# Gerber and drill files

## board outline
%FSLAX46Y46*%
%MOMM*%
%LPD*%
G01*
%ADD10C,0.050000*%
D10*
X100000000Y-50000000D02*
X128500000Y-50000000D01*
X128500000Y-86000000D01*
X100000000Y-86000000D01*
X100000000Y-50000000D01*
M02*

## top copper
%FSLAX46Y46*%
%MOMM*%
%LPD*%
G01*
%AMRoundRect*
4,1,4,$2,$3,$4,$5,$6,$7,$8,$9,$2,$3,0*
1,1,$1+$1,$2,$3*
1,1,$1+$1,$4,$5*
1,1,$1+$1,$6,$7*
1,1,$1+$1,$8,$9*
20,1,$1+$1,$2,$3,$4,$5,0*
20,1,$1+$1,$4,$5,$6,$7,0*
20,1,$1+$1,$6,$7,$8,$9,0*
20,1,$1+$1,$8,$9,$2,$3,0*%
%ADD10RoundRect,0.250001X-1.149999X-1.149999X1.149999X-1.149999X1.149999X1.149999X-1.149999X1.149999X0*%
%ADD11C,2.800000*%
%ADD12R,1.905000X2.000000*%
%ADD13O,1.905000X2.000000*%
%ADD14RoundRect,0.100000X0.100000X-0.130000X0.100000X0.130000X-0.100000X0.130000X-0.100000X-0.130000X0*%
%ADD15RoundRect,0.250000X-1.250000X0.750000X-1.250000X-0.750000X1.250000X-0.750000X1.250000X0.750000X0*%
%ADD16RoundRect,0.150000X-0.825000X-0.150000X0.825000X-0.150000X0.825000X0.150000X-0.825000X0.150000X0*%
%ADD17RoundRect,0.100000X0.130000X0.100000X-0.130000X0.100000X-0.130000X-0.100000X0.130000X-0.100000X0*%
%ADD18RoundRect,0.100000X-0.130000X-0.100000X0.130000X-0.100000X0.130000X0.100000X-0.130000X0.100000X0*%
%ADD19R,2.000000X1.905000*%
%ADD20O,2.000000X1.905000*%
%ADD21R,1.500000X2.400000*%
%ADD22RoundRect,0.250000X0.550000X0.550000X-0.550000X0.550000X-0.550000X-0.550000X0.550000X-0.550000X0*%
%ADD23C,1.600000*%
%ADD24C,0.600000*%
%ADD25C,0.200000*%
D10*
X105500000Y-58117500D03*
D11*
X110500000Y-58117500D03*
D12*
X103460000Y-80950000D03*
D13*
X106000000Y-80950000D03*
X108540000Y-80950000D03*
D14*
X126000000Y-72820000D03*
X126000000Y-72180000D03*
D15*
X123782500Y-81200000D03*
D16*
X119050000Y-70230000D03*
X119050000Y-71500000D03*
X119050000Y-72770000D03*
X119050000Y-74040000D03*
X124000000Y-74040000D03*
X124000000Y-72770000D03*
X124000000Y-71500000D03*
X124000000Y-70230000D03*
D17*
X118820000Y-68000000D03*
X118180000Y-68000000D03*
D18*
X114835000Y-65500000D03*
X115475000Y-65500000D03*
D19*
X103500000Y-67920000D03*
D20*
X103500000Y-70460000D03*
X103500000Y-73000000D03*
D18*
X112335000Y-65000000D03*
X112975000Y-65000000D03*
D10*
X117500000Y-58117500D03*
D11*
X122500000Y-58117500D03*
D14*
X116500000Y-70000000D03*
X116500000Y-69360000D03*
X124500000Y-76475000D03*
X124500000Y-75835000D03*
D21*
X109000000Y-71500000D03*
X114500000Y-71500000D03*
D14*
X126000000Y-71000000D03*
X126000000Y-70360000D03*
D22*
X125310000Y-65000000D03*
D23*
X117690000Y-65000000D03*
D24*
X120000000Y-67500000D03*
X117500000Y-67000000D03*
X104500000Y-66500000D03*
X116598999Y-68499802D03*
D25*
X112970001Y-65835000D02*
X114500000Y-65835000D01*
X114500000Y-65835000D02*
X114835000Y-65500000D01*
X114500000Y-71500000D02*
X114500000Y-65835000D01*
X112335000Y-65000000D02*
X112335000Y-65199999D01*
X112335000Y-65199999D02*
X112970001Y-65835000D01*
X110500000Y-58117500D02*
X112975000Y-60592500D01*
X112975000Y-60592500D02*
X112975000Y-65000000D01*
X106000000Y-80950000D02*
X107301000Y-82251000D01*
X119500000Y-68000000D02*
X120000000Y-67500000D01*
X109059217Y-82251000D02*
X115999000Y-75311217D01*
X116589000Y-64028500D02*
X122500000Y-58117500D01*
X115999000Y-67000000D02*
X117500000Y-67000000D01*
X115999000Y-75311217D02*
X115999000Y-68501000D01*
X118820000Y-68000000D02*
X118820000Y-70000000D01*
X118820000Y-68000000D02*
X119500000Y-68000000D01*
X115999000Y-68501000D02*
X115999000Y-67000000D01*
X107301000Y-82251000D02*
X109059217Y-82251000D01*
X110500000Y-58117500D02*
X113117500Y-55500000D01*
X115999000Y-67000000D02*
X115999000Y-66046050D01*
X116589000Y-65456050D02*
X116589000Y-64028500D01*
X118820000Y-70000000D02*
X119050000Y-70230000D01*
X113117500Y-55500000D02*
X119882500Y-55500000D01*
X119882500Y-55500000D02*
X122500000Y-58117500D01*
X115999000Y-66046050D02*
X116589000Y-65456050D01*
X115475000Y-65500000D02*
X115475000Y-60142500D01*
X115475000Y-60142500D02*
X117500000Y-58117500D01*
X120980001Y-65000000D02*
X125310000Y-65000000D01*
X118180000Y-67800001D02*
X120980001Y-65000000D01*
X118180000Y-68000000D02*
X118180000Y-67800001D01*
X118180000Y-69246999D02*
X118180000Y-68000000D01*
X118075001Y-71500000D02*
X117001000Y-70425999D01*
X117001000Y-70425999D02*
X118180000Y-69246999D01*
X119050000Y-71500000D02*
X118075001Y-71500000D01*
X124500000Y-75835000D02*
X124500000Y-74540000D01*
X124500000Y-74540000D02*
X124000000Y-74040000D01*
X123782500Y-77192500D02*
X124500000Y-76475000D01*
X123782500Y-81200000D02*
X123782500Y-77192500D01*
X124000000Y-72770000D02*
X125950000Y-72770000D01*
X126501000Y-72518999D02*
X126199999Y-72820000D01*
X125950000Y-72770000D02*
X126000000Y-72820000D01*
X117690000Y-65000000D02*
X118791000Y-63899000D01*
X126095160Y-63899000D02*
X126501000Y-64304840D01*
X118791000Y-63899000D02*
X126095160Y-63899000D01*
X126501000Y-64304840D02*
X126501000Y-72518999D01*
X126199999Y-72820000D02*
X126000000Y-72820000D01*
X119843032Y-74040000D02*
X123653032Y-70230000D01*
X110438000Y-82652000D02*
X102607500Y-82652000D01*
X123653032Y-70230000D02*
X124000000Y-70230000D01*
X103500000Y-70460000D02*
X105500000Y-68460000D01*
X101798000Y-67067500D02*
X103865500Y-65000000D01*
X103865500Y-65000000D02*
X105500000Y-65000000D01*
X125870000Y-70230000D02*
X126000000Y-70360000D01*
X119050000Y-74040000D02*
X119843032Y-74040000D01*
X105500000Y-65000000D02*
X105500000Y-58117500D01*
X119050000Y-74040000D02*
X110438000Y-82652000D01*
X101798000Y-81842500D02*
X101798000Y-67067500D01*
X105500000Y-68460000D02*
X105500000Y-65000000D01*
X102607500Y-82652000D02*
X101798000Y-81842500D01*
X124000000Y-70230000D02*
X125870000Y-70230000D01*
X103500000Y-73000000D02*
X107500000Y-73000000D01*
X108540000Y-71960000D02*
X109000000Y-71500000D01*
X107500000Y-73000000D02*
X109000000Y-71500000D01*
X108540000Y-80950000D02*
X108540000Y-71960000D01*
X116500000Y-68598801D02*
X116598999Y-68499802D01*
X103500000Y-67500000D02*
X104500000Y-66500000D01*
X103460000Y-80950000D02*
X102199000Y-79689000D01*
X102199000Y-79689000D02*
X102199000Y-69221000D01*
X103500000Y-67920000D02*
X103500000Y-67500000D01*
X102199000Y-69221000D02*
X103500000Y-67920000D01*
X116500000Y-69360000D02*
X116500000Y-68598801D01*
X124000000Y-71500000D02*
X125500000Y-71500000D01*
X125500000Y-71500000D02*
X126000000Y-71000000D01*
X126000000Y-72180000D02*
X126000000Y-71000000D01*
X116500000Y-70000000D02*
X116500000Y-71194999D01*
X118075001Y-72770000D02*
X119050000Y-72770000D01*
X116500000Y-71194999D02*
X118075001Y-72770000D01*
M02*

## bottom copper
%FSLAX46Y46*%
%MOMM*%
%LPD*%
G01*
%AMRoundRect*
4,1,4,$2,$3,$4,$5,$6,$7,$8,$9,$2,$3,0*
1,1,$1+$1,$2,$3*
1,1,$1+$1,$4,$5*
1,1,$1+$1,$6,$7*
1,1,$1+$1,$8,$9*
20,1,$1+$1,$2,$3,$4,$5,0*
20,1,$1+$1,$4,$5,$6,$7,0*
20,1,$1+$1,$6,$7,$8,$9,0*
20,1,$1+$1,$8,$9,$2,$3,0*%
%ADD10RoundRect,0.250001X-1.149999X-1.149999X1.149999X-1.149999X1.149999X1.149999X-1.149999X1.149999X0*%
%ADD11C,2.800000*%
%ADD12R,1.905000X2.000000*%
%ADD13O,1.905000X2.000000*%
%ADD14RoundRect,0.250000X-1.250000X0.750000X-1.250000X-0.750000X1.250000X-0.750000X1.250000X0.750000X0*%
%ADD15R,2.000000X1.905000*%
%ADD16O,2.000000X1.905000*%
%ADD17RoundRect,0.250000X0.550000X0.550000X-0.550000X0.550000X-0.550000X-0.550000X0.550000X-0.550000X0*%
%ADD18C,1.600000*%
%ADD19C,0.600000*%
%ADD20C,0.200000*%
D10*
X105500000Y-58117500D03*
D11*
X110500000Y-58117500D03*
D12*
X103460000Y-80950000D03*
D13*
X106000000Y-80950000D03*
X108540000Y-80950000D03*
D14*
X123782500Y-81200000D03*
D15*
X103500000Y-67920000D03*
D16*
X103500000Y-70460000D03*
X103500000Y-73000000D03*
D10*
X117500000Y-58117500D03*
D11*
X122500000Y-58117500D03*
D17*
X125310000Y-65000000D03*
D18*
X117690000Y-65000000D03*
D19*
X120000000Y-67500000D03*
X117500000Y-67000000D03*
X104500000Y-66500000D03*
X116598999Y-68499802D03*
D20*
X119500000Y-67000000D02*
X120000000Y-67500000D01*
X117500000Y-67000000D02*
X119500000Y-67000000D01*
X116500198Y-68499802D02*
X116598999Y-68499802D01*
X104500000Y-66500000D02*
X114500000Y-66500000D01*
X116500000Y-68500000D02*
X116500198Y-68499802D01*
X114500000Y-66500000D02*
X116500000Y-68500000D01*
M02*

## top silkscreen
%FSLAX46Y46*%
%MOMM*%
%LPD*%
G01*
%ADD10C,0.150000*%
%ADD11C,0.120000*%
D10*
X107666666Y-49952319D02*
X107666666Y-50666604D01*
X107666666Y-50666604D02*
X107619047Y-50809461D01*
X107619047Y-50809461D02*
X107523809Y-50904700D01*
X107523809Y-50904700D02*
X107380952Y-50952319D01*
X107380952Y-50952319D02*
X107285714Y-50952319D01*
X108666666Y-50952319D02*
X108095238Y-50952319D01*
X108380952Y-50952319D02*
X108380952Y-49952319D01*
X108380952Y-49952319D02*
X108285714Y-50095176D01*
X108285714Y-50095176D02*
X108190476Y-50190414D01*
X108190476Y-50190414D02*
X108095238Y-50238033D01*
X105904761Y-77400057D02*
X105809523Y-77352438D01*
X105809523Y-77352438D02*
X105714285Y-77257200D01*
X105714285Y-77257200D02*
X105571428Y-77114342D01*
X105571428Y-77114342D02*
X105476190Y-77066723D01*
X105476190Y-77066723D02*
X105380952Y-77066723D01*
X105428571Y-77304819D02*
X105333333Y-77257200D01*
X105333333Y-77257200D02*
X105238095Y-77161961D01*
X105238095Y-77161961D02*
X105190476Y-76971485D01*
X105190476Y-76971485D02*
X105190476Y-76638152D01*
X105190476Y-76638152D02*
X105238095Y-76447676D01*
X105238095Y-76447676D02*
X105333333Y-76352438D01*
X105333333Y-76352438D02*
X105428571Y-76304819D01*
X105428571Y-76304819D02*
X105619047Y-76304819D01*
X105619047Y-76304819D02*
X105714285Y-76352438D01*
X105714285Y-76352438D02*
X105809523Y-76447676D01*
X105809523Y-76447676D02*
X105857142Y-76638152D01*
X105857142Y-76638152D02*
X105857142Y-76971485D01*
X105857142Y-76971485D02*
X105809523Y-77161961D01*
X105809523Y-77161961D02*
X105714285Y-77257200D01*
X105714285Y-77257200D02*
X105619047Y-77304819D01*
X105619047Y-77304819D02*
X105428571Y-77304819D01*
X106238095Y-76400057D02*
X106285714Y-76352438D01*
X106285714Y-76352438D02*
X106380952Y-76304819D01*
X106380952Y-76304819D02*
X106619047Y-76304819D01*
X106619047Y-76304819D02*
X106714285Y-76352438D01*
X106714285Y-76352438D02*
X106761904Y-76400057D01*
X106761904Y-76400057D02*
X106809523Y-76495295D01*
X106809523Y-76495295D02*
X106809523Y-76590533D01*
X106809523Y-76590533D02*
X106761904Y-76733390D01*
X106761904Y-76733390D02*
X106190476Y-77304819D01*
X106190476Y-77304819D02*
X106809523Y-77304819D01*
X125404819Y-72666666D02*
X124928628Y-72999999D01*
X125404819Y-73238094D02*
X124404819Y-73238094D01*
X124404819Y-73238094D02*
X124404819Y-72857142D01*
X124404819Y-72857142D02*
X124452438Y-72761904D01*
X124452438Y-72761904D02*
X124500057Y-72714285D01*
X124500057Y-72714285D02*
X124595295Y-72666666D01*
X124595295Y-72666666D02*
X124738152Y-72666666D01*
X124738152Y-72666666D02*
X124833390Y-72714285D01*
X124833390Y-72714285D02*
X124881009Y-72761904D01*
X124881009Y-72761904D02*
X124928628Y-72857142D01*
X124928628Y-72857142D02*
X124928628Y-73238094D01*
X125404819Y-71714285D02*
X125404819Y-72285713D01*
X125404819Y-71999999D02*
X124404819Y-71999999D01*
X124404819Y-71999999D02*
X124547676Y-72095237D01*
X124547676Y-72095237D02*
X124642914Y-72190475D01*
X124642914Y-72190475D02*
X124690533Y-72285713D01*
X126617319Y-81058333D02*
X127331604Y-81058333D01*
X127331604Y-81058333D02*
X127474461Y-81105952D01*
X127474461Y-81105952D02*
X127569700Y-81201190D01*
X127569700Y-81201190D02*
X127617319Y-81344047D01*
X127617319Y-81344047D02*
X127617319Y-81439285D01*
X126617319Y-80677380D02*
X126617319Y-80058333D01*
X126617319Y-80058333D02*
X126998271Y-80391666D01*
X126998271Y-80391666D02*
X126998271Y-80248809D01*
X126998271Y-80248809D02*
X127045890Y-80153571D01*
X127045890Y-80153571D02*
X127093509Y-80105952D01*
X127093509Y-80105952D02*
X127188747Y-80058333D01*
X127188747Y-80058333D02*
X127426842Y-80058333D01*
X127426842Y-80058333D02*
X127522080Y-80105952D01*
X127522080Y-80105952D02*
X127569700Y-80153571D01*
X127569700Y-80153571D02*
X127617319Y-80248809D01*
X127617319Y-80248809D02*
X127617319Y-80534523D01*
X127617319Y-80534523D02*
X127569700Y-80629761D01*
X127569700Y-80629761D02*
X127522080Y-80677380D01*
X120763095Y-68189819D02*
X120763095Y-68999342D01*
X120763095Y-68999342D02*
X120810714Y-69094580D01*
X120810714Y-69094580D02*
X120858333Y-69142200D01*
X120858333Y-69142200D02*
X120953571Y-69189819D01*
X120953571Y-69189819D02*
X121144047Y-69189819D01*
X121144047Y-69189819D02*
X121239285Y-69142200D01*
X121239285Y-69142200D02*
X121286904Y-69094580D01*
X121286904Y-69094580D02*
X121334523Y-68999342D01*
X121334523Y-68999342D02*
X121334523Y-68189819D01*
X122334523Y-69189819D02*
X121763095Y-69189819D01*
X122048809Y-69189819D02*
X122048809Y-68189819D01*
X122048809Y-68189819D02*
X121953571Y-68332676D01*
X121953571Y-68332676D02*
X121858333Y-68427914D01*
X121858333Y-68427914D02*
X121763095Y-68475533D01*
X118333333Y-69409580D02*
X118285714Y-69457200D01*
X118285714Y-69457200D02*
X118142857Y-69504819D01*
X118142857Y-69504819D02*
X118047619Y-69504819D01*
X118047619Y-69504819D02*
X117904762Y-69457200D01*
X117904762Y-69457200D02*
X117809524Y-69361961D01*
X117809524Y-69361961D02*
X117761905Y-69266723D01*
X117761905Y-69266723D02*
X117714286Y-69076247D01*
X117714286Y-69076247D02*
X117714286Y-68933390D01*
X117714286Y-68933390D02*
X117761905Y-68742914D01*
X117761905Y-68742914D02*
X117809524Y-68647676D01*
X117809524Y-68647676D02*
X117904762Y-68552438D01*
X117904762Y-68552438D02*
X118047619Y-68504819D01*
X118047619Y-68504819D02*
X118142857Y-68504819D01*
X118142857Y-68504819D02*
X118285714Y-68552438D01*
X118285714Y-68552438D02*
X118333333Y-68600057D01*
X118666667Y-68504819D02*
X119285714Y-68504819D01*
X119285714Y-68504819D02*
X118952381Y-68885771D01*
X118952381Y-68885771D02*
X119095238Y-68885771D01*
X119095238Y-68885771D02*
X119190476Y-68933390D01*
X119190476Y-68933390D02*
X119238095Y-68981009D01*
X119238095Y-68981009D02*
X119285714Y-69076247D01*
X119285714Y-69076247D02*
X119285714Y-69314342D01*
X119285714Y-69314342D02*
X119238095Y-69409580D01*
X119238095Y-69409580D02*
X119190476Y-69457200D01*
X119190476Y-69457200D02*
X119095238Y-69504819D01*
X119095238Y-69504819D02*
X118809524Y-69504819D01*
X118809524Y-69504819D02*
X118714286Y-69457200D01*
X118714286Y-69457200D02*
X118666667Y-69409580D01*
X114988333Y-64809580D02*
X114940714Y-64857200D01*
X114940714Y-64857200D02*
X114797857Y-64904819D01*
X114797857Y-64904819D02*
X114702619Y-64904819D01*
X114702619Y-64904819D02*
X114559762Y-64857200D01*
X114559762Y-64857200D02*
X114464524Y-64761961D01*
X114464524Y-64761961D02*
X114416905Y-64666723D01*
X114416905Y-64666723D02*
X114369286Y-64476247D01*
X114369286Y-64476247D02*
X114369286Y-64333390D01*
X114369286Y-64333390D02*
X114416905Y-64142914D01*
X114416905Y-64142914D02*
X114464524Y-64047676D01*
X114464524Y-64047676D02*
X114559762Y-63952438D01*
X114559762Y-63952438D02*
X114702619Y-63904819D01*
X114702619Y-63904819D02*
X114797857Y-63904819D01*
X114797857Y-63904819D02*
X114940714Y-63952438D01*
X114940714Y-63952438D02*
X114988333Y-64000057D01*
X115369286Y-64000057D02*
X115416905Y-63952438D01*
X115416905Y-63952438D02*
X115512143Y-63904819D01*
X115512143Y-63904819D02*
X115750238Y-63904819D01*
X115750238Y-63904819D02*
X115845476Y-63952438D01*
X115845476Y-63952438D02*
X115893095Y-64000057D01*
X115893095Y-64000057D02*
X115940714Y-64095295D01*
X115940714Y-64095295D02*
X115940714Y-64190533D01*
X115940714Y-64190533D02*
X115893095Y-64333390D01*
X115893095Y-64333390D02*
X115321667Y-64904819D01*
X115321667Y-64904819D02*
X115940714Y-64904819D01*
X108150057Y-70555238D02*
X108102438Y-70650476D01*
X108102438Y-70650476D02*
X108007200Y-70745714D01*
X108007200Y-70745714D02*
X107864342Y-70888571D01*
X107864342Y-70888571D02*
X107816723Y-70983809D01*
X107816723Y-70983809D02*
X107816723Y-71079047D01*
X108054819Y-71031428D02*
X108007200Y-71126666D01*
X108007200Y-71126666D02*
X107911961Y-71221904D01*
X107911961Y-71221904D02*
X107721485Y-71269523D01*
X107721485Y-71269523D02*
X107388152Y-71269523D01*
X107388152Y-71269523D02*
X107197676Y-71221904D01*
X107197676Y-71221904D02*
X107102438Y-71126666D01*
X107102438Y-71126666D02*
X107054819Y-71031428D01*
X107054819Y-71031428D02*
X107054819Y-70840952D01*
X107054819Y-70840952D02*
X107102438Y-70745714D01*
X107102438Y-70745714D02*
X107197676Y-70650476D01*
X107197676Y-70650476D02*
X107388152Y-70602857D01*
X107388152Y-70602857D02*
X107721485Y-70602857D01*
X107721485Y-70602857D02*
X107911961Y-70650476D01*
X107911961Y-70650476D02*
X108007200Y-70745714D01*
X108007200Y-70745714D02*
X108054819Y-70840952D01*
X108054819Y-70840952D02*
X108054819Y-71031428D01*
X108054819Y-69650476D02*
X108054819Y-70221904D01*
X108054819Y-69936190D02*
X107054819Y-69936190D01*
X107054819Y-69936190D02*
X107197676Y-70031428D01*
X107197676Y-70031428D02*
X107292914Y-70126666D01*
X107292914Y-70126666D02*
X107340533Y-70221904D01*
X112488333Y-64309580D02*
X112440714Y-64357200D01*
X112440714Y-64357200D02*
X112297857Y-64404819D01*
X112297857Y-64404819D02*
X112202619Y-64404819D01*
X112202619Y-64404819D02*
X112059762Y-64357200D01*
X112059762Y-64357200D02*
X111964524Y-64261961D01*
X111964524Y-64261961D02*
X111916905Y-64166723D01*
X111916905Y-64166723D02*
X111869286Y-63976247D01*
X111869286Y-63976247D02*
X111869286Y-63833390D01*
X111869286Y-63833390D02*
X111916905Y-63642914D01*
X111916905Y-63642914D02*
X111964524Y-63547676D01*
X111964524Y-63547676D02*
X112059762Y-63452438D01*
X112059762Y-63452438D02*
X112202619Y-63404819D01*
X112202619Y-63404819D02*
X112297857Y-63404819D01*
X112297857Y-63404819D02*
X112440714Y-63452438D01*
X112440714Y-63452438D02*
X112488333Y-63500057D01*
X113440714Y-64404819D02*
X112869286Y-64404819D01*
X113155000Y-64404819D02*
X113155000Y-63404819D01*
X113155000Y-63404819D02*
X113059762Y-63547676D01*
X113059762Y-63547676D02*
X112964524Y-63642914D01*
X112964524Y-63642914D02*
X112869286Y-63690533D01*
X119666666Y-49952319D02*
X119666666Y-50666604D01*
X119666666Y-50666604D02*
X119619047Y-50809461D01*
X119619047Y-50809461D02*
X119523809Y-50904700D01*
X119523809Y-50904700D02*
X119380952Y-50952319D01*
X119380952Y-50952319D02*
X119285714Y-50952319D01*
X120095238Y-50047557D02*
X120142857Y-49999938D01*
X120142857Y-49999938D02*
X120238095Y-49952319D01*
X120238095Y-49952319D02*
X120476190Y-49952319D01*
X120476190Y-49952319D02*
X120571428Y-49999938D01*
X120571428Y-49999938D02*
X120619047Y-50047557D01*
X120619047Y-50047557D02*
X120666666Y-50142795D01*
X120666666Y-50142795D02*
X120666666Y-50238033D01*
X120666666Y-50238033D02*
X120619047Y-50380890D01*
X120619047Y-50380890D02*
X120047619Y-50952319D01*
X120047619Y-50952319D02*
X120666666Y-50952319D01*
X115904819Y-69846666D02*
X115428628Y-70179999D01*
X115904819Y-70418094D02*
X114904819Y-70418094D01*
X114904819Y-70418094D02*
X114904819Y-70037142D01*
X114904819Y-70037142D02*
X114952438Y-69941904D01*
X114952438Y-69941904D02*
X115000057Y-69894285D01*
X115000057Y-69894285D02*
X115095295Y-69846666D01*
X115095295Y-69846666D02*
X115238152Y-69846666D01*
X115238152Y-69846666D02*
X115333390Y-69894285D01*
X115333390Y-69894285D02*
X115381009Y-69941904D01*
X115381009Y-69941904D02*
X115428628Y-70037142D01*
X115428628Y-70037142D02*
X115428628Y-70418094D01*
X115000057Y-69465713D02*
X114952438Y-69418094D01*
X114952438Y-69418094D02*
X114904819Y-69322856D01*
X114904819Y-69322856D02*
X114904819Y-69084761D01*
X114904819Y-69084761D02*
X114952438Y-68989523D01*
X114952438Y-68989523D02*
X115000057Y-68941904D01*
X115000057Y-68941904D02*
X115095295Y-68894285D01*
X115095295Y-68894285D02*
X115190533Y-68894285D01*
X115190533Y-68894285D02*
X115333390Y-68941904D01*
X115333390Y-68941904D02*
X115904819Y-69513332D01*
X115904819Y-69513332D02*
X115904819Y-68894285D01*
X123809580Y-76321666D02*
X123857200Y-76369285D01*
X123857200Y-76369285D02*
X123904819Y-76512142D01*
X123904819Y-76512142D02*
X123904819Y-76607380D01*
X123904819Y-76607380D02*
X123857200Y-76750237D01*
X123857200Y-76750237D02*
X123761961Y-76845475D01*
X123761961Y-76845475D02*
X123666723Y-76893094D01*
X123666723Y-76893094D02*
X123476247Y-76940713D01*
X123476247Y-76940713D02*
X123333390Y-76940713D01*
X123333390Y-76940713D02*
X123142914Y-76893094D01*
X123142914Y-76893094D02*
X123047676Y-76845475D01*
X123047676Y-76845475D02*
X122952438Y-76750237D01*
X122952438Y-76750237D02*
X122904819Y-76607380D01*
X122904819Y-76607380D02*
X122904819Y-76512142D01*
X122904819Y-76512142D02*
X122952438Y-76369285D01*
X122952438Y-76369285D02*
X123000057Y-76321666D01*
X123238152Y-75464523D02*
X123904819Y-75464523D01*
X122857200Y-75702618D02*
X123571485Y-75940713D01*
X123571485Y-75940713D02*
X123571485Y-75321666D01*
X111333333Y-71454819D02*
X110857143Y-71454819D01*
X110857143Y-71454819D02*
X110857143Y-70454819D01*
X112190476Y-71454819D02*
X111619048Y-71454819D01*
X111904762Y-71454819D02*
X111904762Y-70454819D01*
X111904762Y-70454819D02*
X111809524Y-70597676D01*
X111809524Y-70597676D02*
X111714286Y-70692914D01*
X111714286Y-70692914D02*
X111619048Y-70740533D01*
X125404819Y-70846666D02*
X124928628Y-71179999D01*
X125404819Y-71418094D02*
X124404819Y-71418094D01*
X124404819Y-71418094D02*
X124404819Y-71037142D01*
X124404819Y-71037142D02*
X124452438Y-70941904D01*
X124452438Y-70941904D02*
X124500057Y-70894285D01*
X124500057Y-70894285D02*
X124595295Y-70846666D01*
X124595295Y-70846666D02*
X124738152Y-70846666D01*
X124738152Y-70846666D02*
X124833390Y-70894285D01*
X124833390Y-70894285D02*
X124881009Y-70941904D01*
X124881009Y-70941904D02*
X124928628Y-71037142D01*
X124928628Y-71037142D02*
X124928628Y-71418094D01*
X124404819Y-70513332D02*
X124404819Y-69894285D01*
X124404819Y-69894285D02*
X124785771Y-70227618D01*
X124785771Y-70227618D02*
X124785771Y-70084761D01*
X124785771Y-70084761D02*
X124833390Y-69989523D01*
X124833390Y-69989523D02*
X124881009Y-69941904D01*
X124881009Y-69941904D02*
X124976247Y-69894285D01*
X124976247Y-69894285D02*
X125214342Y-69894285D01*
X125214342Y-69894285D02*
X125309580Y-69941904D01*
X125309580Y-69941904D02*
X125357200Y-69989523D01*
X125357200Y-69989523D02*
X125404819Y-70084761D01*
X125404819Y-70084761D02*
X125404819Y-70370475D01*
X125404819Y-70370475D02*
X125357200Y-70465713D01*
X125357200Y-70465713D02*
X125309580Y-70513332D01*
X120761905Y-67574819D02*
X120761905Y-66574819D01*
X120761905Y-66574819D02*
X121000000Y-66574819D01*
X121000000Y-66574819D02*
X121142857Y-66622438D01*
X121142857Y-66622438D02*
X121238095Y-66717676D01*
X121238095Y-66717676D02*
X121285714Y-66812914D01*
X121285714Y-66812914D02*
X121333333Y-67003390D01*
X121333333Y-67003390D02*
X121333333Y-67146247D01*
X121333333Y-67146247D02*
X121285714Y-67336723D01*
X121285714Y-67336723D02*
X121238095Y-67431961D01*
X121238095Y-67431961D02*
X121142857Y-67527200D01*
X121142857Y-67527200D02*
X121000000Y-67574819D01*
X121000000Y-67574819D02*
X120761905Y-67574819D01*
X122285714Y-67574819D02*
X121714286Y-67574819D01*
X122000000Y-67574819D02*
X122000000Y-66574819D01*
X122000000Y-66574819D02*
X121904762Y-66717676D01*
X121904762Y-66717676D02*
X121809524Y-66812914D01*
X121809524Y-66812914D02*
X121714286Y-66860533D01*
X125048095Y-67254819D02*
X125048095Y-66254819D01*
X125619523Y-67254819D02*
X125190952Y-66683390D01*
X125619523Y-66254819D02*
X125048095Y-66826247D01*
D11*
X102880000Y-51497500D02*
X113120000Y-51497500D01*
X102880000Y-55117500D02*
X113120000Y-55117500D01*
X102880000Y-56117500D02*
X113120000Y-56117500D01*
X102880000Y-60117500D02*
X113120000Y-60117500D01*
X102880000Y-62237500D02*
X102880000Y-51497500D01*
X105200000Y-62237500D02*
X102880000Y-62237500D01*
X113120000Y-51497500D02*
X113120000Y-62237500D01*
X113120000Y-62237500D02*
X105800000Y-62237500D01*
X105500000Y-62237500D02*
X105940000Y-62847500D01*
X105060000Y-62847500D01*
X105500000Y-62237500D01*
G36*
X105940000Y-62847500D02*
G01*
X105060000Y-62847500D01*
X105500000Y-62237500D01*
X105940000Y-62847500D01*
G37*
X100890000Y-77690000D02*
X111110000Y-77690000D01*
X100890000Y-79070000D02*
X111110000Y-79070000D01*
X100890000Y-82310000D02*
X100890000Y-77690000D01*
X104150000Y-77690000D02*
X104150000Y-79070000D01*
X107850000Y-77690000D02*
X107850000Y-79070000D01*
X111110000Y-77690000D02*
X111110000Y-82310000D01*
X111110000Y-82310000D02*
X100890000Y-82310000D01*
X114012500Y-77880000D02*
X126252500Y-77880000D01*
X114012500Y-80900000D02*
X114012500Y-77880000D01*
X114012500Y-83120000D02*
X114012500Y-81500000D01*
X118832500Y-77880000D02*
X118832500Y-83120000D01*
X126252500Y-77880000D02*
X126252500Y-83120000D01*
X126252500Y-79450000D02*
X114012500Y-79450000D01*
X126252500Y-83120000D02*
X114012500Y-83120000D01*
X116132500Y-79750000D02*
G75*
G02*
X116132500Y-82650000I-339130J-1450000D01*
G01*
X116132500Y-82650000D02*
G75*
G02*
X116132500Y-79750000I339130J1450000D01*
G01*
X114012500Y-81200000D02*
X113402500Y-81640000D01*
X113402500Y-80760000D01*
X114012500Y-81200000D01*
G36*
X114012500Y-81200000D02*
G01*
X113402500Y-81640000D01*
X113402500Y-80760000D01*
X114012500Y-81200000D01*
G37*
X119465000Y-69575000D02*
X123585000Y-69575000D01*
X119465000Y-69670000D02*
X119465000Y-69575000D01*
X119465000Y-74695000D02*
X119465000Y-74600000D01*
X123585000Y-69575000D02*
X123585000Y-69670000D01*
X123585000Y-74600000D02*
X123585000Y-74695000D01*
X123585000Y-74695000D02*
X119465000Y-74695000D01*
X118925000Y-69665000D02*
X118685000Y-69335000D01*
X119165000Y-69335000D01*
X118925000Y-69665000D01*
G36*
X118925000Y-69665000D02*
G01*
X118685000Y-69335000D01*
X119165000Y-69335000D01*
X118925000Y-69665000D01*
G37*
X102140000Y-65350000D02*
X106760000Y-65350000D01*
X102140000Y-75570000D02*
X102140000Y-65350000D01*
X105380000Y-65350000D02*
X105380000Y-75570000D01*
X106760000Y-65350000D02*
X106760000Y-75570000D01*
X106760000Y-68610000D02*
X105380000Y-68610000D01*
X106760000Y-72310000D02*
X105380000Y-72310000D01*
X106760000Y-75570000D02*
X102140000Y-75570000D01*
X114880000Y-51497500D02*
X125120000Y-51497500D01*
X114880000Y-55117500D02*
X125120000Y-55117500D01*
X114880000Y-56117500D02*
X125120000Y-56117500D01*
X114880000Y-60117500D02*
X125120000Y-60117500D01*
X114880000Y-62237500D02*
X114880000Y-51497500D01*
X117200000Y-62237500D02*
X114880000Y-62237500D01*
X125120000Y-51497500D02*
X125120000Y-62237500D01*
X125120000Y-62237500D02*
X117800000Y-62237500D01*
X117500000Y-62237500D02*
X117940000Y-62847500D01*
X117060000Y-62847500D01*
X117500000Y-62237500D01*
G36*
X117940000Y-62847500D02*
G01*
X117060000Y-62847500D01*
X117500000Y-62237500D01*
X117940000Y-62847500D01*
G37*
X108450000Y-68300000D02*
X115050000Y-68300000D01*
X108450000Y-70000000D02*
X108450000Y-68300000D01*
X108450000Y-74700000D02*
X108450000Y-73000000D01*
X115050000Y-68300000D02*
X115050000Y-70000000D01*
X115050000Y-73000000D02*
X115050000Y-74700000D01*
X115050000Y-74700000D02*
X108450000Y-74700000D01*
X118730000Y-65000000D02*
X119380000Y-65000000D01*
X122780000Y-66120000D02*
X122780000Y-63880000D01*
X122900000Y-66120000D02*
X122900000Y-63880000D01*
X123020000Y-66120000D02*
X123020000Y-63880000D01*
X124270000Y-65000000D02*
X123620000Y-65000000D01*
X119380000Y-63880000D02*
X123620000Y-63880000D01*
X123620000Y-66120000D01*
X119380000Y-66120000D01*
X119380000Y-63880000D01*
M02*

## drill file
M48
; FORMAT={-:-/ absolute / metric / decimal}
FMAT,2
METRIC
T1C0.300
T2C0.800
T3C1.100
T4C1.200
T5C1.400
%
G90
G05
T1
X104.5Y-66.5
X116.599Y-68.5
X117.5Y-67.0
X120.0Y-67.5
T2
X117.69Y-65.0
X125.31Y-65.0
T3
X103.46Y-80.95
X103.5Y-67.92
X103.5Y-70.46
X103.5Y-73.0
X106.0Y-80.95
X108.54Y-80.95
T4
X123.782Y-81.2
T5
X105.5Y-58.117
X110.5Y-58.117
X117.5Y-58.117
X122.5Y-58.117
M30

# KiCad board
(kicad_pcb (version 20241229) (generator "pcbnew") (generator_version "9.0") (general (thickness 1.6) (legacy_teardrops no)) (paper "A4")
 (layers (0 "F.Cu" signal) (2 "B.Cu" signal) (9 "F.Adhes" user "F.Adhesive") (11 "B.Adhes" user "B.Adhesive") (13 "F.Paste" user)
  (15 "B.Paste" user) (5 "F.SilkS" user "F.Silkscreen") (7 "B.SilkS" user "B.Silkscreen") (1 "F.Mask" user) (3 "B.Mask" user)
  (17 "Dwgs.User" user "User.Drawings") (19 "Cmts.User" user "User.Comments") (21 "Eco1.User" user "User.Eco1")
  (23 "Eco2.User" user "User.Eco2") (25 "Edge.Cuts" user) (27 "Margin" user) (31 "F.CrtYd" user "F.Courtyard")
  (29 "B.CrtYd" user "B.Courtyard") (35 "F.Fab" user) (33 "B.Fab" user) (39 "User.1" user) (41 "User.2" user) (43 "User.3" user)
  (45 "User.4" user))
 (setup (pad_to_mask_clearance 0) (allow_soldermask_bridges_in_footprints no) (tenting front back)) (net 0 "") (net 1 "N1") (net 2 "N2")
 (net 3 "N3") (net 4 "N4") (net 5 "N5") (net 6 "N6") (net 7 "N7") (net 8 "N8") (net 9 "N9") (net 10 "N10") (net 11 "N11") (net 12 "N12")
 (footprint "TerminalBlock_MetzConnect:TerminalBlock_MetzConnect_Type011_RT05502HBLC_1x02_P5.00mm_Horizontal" (layer "F.Cu")
  (at 105.5 58.1175)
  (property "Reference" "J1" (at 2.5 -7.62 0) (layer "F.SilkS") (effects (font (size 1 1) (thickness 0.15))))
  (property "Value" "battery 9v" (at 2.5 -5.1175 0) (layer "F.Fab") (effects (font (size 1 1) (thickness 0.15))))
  (fp_line (start -2.62 -6.62) (end 7.62 -6.62) (stroke (width 0.12) (type solid)) (layer "F.SilkS"))
  (fp_line (start -2.62 -3) (end 7.62 -3) (stroke (width 0.12) (type solid)) (layer "F.SilkS"))
  (fp_line (start -2.62 -2) (end 7.62 -2) (stroke (width 0.12) (type solid)) (layer "F.SilkS"))
  (fp_line (start -2.62 2) (end 7.62 2) (stroke (width 0.12) (type solid)) (layer "F.SilkS"))
  (fp_line (start -2.62 4.12) (end -2.62 -6.62) (stroke (width 0.12) (type solid)) (layer "F.SilkS"))
  (fp_line (start -0.3 4.12) (end -2.62 4.12) (stroke (width 0.12) (type solid)) (layer "F.SilkS"))
  (fp_line (start 7.62 -6.62) (end 7.62 4.12) (stroke (width 0.12) (type solid)) (layer "F.SilkS"))
  (fp_line (start 7.62 4.12) (end 0.3 4.12) (stroke (width 0.12) (type solid)) (layer "F.SilkS"))
  (fp_poly (pts (xy 0 4.12) (xy 0.44 4.73) (xy -0.44 4.73)) (stroke (width 0.12) (type solid)) (fill yes) (layer "F.SilkS"))
  (pad "1" thru_hole roundrect (at 0 0) (size 2.8 2.8) (drill 1.4) (layers "*.Cu" "*.Mask") (remove_unused_layers no)
   (roundrect_rratio 0.089286) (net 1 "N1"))
  (pad "2" thru_hole circle (at 5 0) (size 2.8 2.8) (drill 1.4) (layers "*.Cu" "*.Mask") (remove_unused_layers no) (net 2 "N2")))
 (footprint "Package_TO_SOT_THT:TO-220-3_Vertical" (layer "F.Cu") (at 103.46 80.95)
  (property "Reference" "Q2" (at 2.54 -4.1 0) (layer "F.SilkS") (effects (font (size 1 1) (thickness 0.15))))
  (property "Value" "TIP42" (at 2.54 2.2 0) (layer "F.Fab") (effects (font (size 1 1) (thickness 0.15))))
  (fp_line (start -2.57 -3.26) (end 7.65 -3.26) (stroke (width 0.12) (type solid)) (layer "F.SilkS"))
  (fp_line (start -2.57 -1.88) (end 7.65 -1.88) (stroke (width 0.12) (type solid)) (layer "F.SilkS"))
  (fp_line (start -2.57 1.36) (end -2.57 -3.26) (stroke (width 0.12) (type solid)) (layer "F.SilkS"))
  (fp_line (start 0.69 -3.26) (end 0.69 -1.88) (stroke (width 0.12) (type solid)) (layer "F.SilkS"))
  (fp_line (start 4.39 -3.26) (end 4.39 -1.88) (stroke (width 0.12) (type solid)) (layer "F.SilkS"))
  (fp_line (start 7.65 -3.26) (end 7.65 1.36) (stroke (width 0.12) (type solid)) (layer "F.SilkS"))
  (fp_line (start 7.65 1.36) (end -2.57 1.36) (stroke (width 0.12) (type solid)) (layer "F.SilkS"))
  (pad "1" thru_hole rect (at 0 0) (size 1.905 2) (drill 1.1) (layers "*.Cu" "*.Mask") (remove_unused_layers no) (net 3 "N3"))
  (pad "2" thru_hole oval (at 2.54 0) (size 1.905 2) (drill 1.1) (layers "*.Cu" "*.Mask") (remove_unused_layers no) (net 2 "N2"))
  (pad "3" thru_hole oval (at 5.08 0) (size 1.905 2) (drill 1.1) (layers "*.Cu" "*.Mask") (remove_unused_layers no) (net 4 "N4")))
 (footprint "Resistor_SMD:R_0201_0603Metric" (layer "F.Cu") (at 126 72.5 90)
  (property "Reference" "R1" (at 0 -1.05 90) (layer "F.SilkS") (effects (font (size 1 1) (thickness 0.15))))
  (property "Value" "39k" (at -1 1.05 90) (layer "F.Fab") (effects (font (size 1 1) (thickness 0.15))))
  (pad "" smd roundrect (at -0.345 0 90) (size 0.318 0.36) (layers "F.Paste") (roundrect_rratio 0.25))
  (pad "" smd roundrect (at 0.345 0 90) (size 0.318 0.36) (layers "F.Paste") (roundrect_rratio 0.25))
  (pad "1" smd roundrect (at -0.32 0 90) (size 0.46 0.4) (layers "F.Cu" "F.Mask") (roundrect_rratio 0.25) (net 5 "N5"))
  (pad "2" smd roundrect (at 0.32 0 90) (size 0.46 0.4) (layers "F.Cu" "F.Mask") (roundrect_rratio 0.25) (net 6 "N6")))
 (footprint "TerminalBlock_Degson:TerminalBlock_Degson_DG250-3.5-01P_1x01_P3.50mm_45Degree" (layer "F.Cu") (at 123.7825 81.2 -90)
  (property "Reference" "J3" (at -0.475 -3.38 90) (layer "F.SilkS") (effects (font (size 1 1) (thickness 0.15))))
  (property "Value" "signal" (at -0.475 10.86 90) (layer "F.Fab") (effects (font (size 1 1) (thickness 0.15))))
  (fp_line (start -3.32 9.77) (end -3.32 -2.47) (stroke (width 0.12) (type solid)) (layer "F.SilkS"))
  (fp_line (start -0.3 9.77) (end -3.32 9.77) (stroke (width 0.12) (type solid)) (layer "F.SilkS"))
  (fp_line (start 1.92 9.77) (end 0.3 9.77) (stroke (width 0.12) (type solid)) (layer "F.SilkS"))
  (fp_line (start -3.32 4.95) (end 1.92 4.95) (stroke (width 0.12) (type solid)) (layer "F.SilkS"))
  (fp_line (start -3.32 -2.47) (end 1.92 -2.47) (stroke (width 0.12) (type solid)) (layer "F.SilkS"))
  (fp_line (start -1.75 -2.47) (end -1.75 9.77) (stroke (width 0.12) (type solid)) (layer "F.SilkS"))
  (fp_line (start 1.92 -2.47) (end 1.92 9.77) (stroke (width 0.12) (type solid)) (layer "F.SilkS"))
  (fp_arc (start -1.45 7.65) (mid 0 6.5) (end 1.45 7.65) (stroke (width 0.12) (type solid)) (layer "F.SilkS"))
  (fp_arc (start 1.45 7.65) (mid 0 8.8) (end -1.45 7.65) (stroke (width 0.12) (type solid)) (layer "F.SilkS"))
  (fp_poly (pts (xy 0 9.77) (xy 0.44 10.38) (xy -0.44 10.38)) (stroke (width 0.12) (type solid)) (fill yes) (layer "F.SilkS"))
  (pad "1" thru_hole roundrect (at 0 0 270) (size 2 3) (drill 1.2) (layers "*.Cu" "*.Mask") (remove_unused_layers no)
   (roundrect_rratio 0.125) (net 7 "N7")))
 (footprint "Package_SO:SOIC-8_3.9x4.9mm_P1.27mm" (layer "F.Cu") (at 121.525 72.135)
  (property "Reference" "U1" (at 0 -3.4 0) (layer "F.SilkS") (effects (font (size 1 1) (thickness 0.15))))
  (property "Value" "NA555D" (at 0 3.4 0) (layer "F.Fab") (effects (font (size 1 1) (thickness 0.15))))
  (fp_line (start -2.06 -2.56) (end 2.06 -2.56) (stroke (width 0.12) (type solid)) (layer "F.SilkS"))
  (fp_line (start -2.06 -2.465) (end -2.06 -2.56) (stroke (width 0.12) (type solid)) (layer "F.SilkS"))
  (fp_line (start -2.06 2.56) (end -2.06 2.465) (stroke (width 0.12) (type solid)) (layer "F.SilkS"))
  (fp_line (start 2.06 -2.56) (end 2.06 -2.465) (stroke (width 0.12) (type solid)) (layer "F.SilkS"))
  (fp_line (start 2.06 2.465) (end 2.06 2.56) (stroke (width 0.12) (type solid)) (layer "F.SilkS"))
  (fp_line (start 2.06 2.56) (end -2.06 2.56) (stroke (width 0.12) (type solid)) (layer "F.SilkS"))
  (fp_poly (pts (xy -2.6 -2.47) (xy -2.84 -2.8) (xy -2.36 -2.8)) (stroke (width 0.12) (type solid)) (fill yes) (layer "F.SilkS"))
  (pad "1" smd roundrect (at -2.475 -1.905) (size 1.95 0.6) (layers "F.Cu" "F.Mask" "F.Paste") (roundrect_rratio 0.25) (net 2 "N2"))
  (pad "2" smd roundrect (at -2.475 -0.635) (size 1.95 0.6) (layers "F.Cu" "F.Mask" "F.Paste") (roundrect_rratio 0.25) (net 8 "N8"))
  (pad "3" smd roundrect (at -2.475 0.635) (size 1.95 0.6) (layers "F.Cu" "F.Mask" "F.Paste") (roundrect_rratio 0.25) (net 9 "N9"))
  (pad "4" smd roundrect (at -2.475 1.905) (size 1.95 0.6) (layers "F.Cu" "F.Mask" "F.Paste") (roundrect_rratio 0.25) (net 1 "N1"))
  (pad "5" smd roundrect (at 2.475 1.905) (size 1.95 0.6) (layers "F.Cu" "F.Mask" "F.Paste") (roundrect_rratio 0.25) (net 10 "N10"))
  (pad "6" smd roundrect (at 2.475 0.635) (size 1.95 0.6) (layers "F.Cu" "F.Mask" "F.Paste") (roundrect_rratio 0.25) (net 5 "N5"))
  (pad "7" smd roundrect (at 2.475 -0.635) (size 1.95 0.6) (layers "F.Cu" "F.Mask" "F.Paste") (roundrect_rratio 0.25) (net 6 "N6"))
  (pad "8" smd roundrect (at 2.475 -1.905) (size 1.95 0.6) (layers "F.Cu" "F.Mask" "F.Paste") (roundrect_rratio 0.25) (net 1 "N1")))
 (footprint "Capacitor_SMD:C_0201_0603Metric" (layer "F.Cu") (at 118.5 68 180)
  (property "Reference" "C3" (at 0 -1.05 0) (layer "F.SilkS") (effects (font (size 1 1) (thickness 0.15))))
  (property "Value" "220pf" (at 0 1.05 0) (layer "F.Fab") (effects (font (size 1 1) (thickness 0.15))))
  (pad "" smd roundrect (at -0.345 0 180) (size 0.318 0.36) (layers "F.Paste") (roundrect_rratio 0.25))
  (pad "" smd roundrect (at 0.345 0 180) (size 0.318 0.36) (layers "F.Paste") (roundrect_rratio 0.25))
  (pad "1" smd roundrect (at -0.32 0 180) (size 0.46 0.4) (layers "F.Cu" "F.Mask") (roundrect_rratio 0.25) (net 2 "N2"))
  (pad "2" smd roundrect (at 0.32 0 180) (size 0.46 0.4) (layers "F.Cu" "F.Mask") (roundrect_rratio 0.25) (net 8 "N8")))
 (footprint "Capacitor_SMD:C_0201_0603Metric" (layer "F.Cu") (at 115.155 65.5)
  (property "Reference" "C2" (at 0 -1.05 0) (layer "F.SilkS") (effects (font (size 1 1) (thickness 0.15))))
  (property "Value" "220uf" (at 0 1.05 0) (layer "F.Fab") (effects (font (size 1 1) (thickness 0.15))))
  (pad "" smd roundrect (at -0.345 0) (size 0.318 0.36) (layers "F.Paste") (roundrect_rratio 0.25))
  (pad "" smd roundrect (at 0.345 0) (size 0.318 0.36) (layers "F.Paste") (roundrect_rratio 0.25))
  (pad "1" smd roundrect (at -0.32 0) (size 0.46 0.4) (layers "F.Cu" "F.Mask") (roundrect_rratio 0.25) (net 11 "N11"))
  (pad "2" smd roundrect (at 0.32 0) (size 0.46 0.4) (layers "F.Cu" "F.Mask") (roundrect_rratio 0.25) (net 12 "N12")))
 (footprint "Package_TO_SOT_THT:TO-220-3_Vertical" (layer "F.Cu") (at 103.5 67.92 -90)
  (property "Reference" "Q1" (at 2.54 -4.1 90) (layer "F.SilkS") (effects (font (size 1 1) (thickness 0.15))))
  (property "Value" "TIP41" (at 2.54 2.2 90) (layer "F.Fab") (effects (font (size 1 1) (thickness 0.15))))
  (fp_line (start -2.57 1.36) (end -2.57 -3.26) (stroke (width 0.12) (type solid)) (layer "F.SilkS"))
  (fp_line (start 7.65 1.36) (end -2.57 1.36) (stroke (width 0.12) (type solid)) (layer "F.SilkS"))
  (fp_line (start -2.57 -1.88) (end 7.65 -1.88) (stroke (width 0.12) (type solid)) (layer "F.SilkS"))
  (fp_line (start -2.57 -3.26) (end 7.65 -3.26) (stroke (width 0.12) (type solid)) (layer "F.SilkS"))
  (fp_line (start 0.69 -3.26) (end 0.69 -1.88) (stroke (width 0.12) (type solid)) (layer "F.SilkS"))
  (fp_line (start 4.39 -3.26) (end 4.39 -1.88) (stroke (width 0.12) (type solid)) (layer "F.SilkS"))
  (fp_line (start 7.65 -3.26) (end 7.65 1.36) (stroke (width 0.12) (type solid)) (layer "F.SilkS"))
  (pad "1" thru_hole rect (at 0 0 270) (size 1.905 2) (drill 1.1) (layers "*.Cu" "*.Mask") (remove_unused_layers no) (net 3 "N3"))
  (pad "2" thru_hole oval (at 2.54 0 270) (size 1.905 2) (drill 1.1) (layers "*.Cu" "*.Mask") (remove_unused_layers no) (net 1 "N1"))
  (pad "3" thru_hole oval (at 5.08 0 270) (size 1.905 2) (drill 1.1) (layers "*.Cu" "*.Mask") (remove_unused_layers no) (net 4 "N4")))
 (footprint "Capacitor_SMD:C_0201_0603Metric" (layer "F.Cu") (at 112.655 65)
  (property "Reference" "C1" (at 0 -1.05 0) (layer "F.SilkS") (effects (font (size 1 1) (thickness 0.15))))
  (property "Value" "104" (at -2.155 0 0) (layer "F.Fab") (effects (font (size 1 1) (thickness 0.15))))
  (pad "" smd roundrect (at -0.345 0) (size 0.318 0.36) (layers "F.Paste") (roundrect_rratio 0.25))
  (pad "" smd roundrect (at 0.345 0) (size 0.318 0.36) (layers "F.Paste") (roundrect_rratio 0.25))
  (pad "1" smd roundrect (at -0.32 0) (size 0.46 0.4) (layers "F.Cu" "F.Mask") (roundrect_rratio 0.25) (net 11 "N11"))
  (pad "2" smd roundrect (at 0.32 0) (size 0.46 0.4) (layers "F.Cu" "F.Mask") (roundrect_rratio 0.25) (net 2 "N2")))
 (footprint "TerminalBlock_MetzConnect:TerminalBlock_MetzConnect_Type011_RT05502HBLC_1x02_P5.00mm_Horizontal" (layer "F.Cu")
  (at 117.5 58.1175)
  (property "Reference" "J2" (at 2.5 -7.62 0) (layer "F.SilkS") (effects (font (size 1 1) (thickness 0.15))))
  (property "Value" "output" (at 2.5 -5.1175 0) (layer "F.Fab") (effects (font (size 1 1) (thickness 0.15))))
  (fp_line (start -2.62 -6.62) (end 7.62 -6.62) (stroke (width 0.12) (type solid)) (layer "F.SilkS"))
  (fp_line (start -2.62 -3) (end 7.62 -3) (stroke (width 0.12) (type solid)) (layer "F.SilkS"))
  (fp_line (start -2.62 -2) (end 7.62 -2) (stroke (width 0.12) (type solid)) (layer "F.SilkS"))
  (fp_line (start -2.62 2) (end 7.62 2) (stroke (width 0.12) (type solid)) (layer "F.SilkS"))
  (fp_line (start -2.62 4.12) (end -2.62 -6.62) (stroke (width 0.12) (type solid)) (layer "F.SilkS"))
  (fp_line (start -0.3 4.12) (end -2.62 4.12) (stroke (width 0.12) (type solid)) (layer "F.SilkS"))
  (fp_line (start 7.62 -6.62) (end 7.62 4.12) (stroke (width 0.12) (type solid)) (layer "F.SilkS"))
  (fp_line (start 7.62 4.12) (end 0.3 4.12) (stroke (width 0.12) (type solid)) (layer "F.SilkS"))
  (fp_poly (pts (xy 0 4.12) (xy 0.44 4.73) (xy -0.44 4.73)) (stroke (width 0.12) (type solid)) (fill yes) (layer "F.SilkS"))
  (pad "1" thru_hole roundrect (at 0 0) (size 2.8 2.8) (drill 1.4) (layers "*.Cu" "*.Mask") (remove_unused_layers no)
   (roundrect_rratio 0.089286) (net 12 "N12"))
  (pad "2" thru_hole circle (at 5 0) (size 2.8 2.8) (drill 1.4) (layers "*.Cu" "*.Mask") (remove_unused_layers no) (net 2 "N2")))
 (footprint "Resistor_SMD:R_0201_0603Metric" (layer "F.Cu") (at 116.5 69.68 90)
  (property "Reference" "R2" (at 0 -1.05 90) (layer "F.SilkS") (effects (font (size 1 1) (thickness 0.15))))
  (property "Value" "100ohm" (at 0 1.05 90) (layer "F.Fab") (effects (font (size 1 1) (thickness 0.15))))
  (pad "" smd roundrect (at -0.345 0 90) (size 0.318 0.36) (layers "F.Paste") (roundrect_rratio 0.25))
  (pad "" smd roundrect (at 0.345 0 90) (size 0.318 0.36) (layers "F.Paste") (roundrect_rratio 0.25))
  (pad "1" smd roundrect (at -0.32 0 90) (size 0.46 0.4) (layers "F.Cu" "F.Mask") (roundrect_rratio 0.25) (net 9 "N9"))
  (pad "2" smd roundrect (at 0.32 0 90) (size 0.46 0.4) (layers "F.Cu" "F.Mask") (roundrect_rratio 0.25) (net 3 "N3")))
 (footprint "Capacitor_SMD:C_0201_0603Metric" (layer "F.Cu") (at 124.5 76.155 90)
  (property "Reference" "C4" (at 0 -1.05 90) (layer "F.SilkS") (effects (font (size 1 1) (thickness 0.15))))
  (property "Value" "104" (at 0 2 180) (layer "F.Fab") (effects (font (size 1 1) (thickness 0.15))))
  (pad "" smd roundrect (at -0.345 0 90) (size 0.318 0.36) (layers "F.Paste") (roundrect_rratio 0.25))
  (pad "" smd roundrect (at 0.345 0 90) (size 0.318 0.36) (layers "F.Paste") (roundrect_rratio 0.25))
  (pad "1" smd roundrect (at -0.32 0 90) (size 0.46 0.4) (layers "F.Cu" "F.Mask") (roundrect_rratio 0.25) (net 7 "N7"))
  (pad "2" smd roundrect (at 0.32 0 90) (size 0.46 0.4) (layers "F.Cu" "F.Mask") (roundrect_rratio 0.25) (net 10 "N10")))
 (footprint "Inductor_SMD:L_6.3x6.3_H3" (layer "F.Cu") (at 111.75 71.5)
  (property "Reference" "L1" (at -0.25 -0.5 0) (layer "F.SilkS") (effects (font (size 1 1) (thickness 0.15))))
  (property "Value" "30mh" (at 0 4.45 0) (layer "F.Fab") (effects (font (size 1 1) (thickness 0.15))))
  (fp_line (start -3.3 -3.2) (end 3.3 -3.2) (stroke (width 0.12) (type solid)) (layer "F.SilkS"))
  (fp_line (start -3.3 -1.5) (end -3.3 -3.2) (stroke (width 0.12) (type solid)) (layer "F.SilkS"))
  (fp_line (start -3.3 3.2) (end -3.3 1.5) (stroke (width 0.12) (type solid)) (layer "F.SilkS"))
  (fp_line (start 3.3 -3.2) (end 3.3 -1.5) (stroke (width 0.12) (type solid)) (layer "F.SilkS"))
  (fp_line (start 3.3 1.5) (end 3.3 3.2) (stroke (width 0.12) (type solid)) (layer "F.SilkS"))
  (fp_line (start 3.3 3.2) (end -3.3 3.2) (stroke (width 0.12) (type solid)) (layer "F.SilkS"))
  (pad "1" smd rect (at -2.75 0) (size 1.5 2.4) (layers "F.Cu" "F.Mask" "F.Paste") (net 4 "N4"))
  (pad "2" smd rect (at 2.75 0) (size 1.5 2.4) (layers "F.Cu" "F.Mask" "F.Paste") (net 11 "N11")))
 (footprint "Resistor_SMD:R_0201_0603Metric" (layer "F.Cu") (at 126 70.68 90)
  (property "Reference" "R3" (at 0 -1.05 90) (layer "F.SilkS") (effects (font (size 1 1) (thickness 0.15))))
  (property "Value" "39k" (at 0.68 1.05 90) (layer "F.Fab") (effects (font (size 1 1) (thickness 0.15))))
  (pad "" smd roundrect (at -0.345 0 90) (size 0.318 0.36) (layers "F.Paste") (roundrect_rratio 0.25))
  (pad "" smd roundrect (at 0.345 0 90) (size 0.318 0.36) (layers "F.Paste") (roundrect_rratio 0.25))
  (pad "1" smd roundrect (at -0.32 0 90) (size 0.46 0.4) (layers "F.Cu" "F.Mask") (roundrect_rratio 0.25) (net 6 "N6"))
  (pad "2" smd roundrect (at 0.32 0 90) (size 0.46 0.4) (layers "F.Cu" "F.Mask") (roundrect_rratio 0.25) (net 1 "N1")))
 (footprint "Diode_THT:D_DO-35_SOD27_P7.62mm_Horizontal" (layer "F.Cu") (at 125.31 65 180)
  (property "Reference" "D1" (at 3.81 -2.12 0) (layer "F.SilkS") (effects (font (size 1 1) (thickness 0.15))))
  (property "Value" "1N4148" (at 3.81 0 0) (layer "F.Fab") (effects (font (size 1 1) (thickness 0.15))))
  (fp_line (start 6.58 0) (end 5.93 0) (stroke (width 0.12) (type solid)) (layer "F.SilkS"))
  (fp_line (start 2.53 -1.12) (end 2.53 1.12) (stroke (width 0.12) (type solid)) (layer "F.SilkS"))
  (fp_line (start 2.41 -1.12) (end 2.41 1.12) (stroke (width 0.12) (type solid)) (layer "F.SilkS"))
  (fp_line (start 2.29 -1.12) (end 2.29 1.12) (stroke (width 0.12) (type solid)) (layer "F.SilkS"))
  (fp_line (start 1.04 0) (end 1.69 0) (stroke (width 0.12) (type solid)) (layer "F.SilkS"))
  (fp_rect (start 1.69 -1.12) (end 5.93 1.12) (stroke (width 0.12) (type solid)) (fill no) (layer "F.SilkS"))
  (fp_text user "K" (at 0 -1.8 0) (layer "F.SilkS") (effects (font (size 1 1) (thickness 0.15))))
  (pad "1" thru_hole roundrect (at 0 0 180) (size 1.6 1.6) (drill 0.8) (layers "*.Cu" "*.Mask") (remove_unused_layers no)
   (roundrect_rratio 0.15625) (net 8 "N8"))
  (pad "2" thru_hole circle (at 7.62 0 180) (size 1.6 1.6) (drill 0.8) (layers "*.Cu" "*.Mask") (remove_unused_layers no) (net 5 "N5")))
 (gr_rect (start 100 50) (end 128.5 86) (stroke (width 0.05) (type default)) (fill no) (layer "Edge.Cuts"))
 (segment (start 112.970001 65.835) (end 114.5 65.835) (width 0.2) (layer "F.Cu") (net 11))
 (segment (start 114.5 65.835) (end 114.835 65.5) (width 0.2) (layer "F.Cu") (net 11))
 (segment (start 114.5 71.5) (end 114.5 65.835) (width 0.2) (layer "F.Cu") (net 11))
 (segment (start 112.335 65) (end 112.335 65.199999) (width 0.2) (layer "F.Cu") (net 11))
 (segment (start 112.335 65.199999) (end 112.970001 65.835) (width 0.2) (layer "F.Cu") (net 11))
 (segment (start 110.5 58.1175) (end 112.975 60.5925) (width 0.2) (layer "F.Cu") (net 2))
 (segment (start 112.975 60.5925) (end 112.975 65) (width 0.2) (layer "F.Cu") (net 2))
 (segment (start 106 80.95) (end 107.301 82.251) (width 0.2) (layer "F.Cu") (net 2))
 (segment (start 119.5 68) (end 120 67.5) (width 0.2) (layer "F.Cu") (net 2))
 (segment (start 109.059217 82.251) (end 115.999 75.311217) (width 0.2) (layer "F.Cu") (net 2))
 (segment (start 116.589 64.0285) (end 122.5 58.1175) (width 0.2) (layer "F.Cu") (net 2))
 (segment (start 115.999 67) (end 117.5 67) (width 0.2) (layer "F.Cu") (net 2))
 (segment (start 115.999 75.311217) (end 115.999 68.501) (width 0.2) (layer "F.Cu") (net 2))
 (segment (start 118.82 68) (end 118.82 70) (width 0.2) (layer "F.Cu") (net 2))
 (segment (start 118.82 68) (end 119.5 68) (width 0.2) (layer "F.Cu") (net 2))
 (segment (start 115.999 68.501) (end 115.999 67) (width 0.2) (layer "F.Cu") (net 2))
 (segment (start 107.301 82.251) (end 109.059217 82.251) (width 0.2) (layer "F.Cu") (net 2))
 (segment (start 110.5 58.1175) (end 113.1175 55.5) (width 0.2) (layer "F.Cu") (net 2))
 (segment (start 115.999 67) (end 115.999 66.04605) (width 0.2) (layer "F.Cu") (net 2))
 (segment (start 116.589 65.45605) (end 116.589 64.0285) (width 0.2) (layer "F.Cu") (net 2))
 (segment (start 118.82 70) (end 119.05 70.23) (width 0.2) (layer "F.Cu") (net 2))
 (segment (start 113.1175 55.5) (end 119.8825 55.5) (width 0.2) (layer "F.Cu") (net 2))
 (segment (start 119.8825 55.5) (end 122.5 58.1175) (width 0.2) (layer "F.Cu") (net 2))
 (segment (start 115.999 66.04605) (end 116.589 65.45605) (width 0.2) (layer "F.Cu") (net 2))
 (via (at 120 67.5) (size 0.6) (drill 0.3) (layers "F.Cu" "B.Cu") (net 2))
 (via (at 117.5 67) (size 0.6) (drill 0.3) (layers "F.Cu" "B.Cu") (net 2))
 (segment (start 119.5 67) (end 120 67.5) (width 0.2) (layer "B.Cu") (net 2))
 (segment (start 117.5 67) (end 119.5 67) (width 0.2) (layer "B.Cu") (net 2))
 (segment (start 115.475 65.5) (end 115.475 60.1425) (width 0.2) (layer "F.Cu") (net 12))
 (segment (start 115.475 60.1425) (end 117.5 58.1175) (width 0.2) (layer "F.Cu") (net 12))
 (segment (start 120.980001 65) (end 125.31 65) (width 0.2) (layer "F.Cu") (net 8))
 (segment (start 118.18 67.800001) (end 120.980001 65) (width 0.2) (layer "F.Cu") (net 8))
 (segment (start 118.18 68) (end 118.18 67.800001) (width 0.2) (layer "F.Cu") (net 8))
 (segment (start 118.18 69.246999) (end 118.18 68) (width 0.2) (layer "F.Cu") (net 8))
 (segment (start 118.075001 71.5) (end 117.001 70.425999) (width 0.2) (layer "F.Cu") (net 8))
 (segment (start 117.001 70.425999) (end 118.18 69.246999) (width 0.2) (layer "F.Cu") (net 8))
 (segment (start 119.05 71.5) (end 118.075001 71.5) (width 0.2) (layer "F.Cu") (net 8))
 (segment (start 124.5 75.835) (end 124.5 74.54) (width 0.2) (layer "F.Cu") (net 10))
 (segment (start 124.5 74.54) (end 124 74.04) (width 0.2) (layer "F.Cu") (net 10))
 (segment (start 123.7825 77.1925) (end 124.5 76.475) (width 0.2) (layer "F.Cu") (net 7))
 (segment (start 123.7825 81.2) (end 123.7825 77.1925) (width 0.2) (layer "F.Cu") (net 7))
 (segment (start 124 72.77) (end 125.95 72.77) (width 0.2) (layer "F.Cu") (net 5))
 (segment (start 126.501 72.518999) (end 126.199999 72.82) (width 0.2) (layer "F.Cu") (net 5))
 (segment (start 125.95 72.77) (end 126 72.82) (width 0.2) (layer "F.Cu") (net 5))
 (segment (start 117.69 65) (end 118.791 63.899) (width 0.2) (layer "F.Cu") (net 5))
 (segment (start 126.09516 63.899) (end 126.501 64.30484) (width 0.2) (layer "F.Cu") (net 5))
 (segment (start 118.791 63.899) (end 126.09516 63.899) (width 0.2) (layer "F.Cu") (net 5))
 (segment (start 126.501 64.30484) (end 126.501 72.518999) (width 0.2) (layer "F.Cu") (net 5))
 (segment (start 126.199999 72.82) (end 126 72.82) (width 0.2) (layer "F.Cu") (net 5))
 (segment (start 119.843032 74.04) (end 123.653032 70.23) (width 0.2) (layer "F.Cu") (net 1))
 (segment (start 110.438 82.652) (end 102.6075 82.652) (width 0.2) (layer "F.Cu") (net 1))
 (segment (start 123.653032 70.23) (end 124 70.23) (width 0.2) (layer "F.Cu") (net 1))
 (segment (start 103.5 70.46) (end 105.5 68.46) (width 0.2) (layer "F.Cu") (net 1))
 (segment (start 101.798 67.0675) (end 103.8655 65) (width 0.2) (layer "F.Cu") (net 1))
 (segment (start 103.8655 65) (end 105.5 65) (width 0.2) (layer "F.Cu") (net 1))
 (segment (start 125.87 70.23) (end 126 70.36) (width 0.2) (layer "F.Cu") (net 1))
 (segment (start 119.05 74.04) (end 119.843032 74.04) (width 0.2) (layer "F.Cu") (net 1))
 (segment (start 105.5 65) (end 105.5 58.1175) (width 0.2) (layer "F.Cu") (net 1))
 (segment (start 119.05 74.04) (end 110.438 82.652) (width 0.2) (layer "F.Cu") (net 1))
 (segment (start 101.798 81.8425) (end 101.798 67.0675) (width 0.2) (layer "F.Cu") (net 1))
 (segment (start 105.5 68.46) (end 105.5 65) (width 0.2) (layer "F.Cu") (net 1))
 (segment (start 102.6075 82.652) (end 101.798 81.8425) (width 0.2) (layer "F.Cu") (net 1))
 (segment (start 124 70.23) (end 125.87 70.23) (width 0.2) (layer "F.Cu") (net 1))
 (segment (start 103.5 73) (end 107.5 73) (width 0.2) (layer "F.Cu") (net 4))
 (segment (start 108.54 71.96) (end 109 71.5) (width 0.2) (layer "F.Cu") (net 4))
 (segment (start 107.5 73) (end 109 71.5) (width 0.2) (layer "F.Cu") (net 4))
 (segment (start 108.54 80.95) (end 108.54 71.96) (width 0.2) (layer "F.Cu") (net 4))
 (segment (start 116.5 68.598801) (end 116.598999 68.499802) (width 0.2) (layer "F.Cu") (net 3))
 (segment (start 103.5 67.5) (end 104.5 66.5) (width 0.2) (layer "F.Cu") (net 3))
 (segment (start 103.46 80.95) (end 102.199 79.689) (width 0.2) (layer "F.Cu") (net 3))
 (segment (start 102.199 79.689) (end 102.199 69.221) (width 0.2) (layer "F.Cu") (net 3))
 (segment (start 103.5 67.92) (end 103.5 67.5) (width 0.2) (layer "F.Cu") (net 3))
 (segment (start 102.199 69.221) (end 103.5 67.92) (width 0.2) (layer "F.Cu") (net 3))
 (segment (start 116.5 69.36) (end 116.5 68.598801) (width 0.2) (layer "F.Cu") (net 3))
 (via (at 104.5 66.5) (size 0.6) (drill 0.3) (layers "F.Cu" "B.Cu") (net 3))
 (via (at 116.598999 68.499802) (size 0.6) (drill 0.3) (layers "F.Cu" "B.Cu") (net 3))
 (segment (start 116.500198 68.499802) (end 116.598999 68.499802) (width 0.2) (layer "B.Cu") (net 3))
 (segment (start 104.5 66.5) (end 114.5 66.5) (width 0.2) (layer "B.Cu") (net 3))
 (segment (start 116.5 68.5) (end 116.500198 68.499802) (width 0.2) (layer "B.Cu") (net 3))
 (segment (start 114.5 66.5) (end 116.5 68.5) (width 0.2) (layer "B.Cu") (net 3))
 (segment (start 124 71.5) (end 125.5 71.5) (width 0.2) (layer "F.Cu") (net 6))
 (segment (start 125.5 71.5) (end 126 71) (width 0.2) (layer "F.Cu") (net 6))
 (segment (start 126 72.18) (end 126 71) (width 0.2) (layer "F.Cu") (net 6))
 (segment (start 116.5 70) (end 116.5 71.194999) (width 0.2) (layer "F.Cu") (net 9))
 (segment (start 118.075001 72.77) (end 119.05 72.77) (width 0.2) (layer "F.Cu") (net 9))
 (segment (start 116.5 71.194999) (end 118.075001 72.77) (width 0.2) (layer "F.Cu") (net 9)))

